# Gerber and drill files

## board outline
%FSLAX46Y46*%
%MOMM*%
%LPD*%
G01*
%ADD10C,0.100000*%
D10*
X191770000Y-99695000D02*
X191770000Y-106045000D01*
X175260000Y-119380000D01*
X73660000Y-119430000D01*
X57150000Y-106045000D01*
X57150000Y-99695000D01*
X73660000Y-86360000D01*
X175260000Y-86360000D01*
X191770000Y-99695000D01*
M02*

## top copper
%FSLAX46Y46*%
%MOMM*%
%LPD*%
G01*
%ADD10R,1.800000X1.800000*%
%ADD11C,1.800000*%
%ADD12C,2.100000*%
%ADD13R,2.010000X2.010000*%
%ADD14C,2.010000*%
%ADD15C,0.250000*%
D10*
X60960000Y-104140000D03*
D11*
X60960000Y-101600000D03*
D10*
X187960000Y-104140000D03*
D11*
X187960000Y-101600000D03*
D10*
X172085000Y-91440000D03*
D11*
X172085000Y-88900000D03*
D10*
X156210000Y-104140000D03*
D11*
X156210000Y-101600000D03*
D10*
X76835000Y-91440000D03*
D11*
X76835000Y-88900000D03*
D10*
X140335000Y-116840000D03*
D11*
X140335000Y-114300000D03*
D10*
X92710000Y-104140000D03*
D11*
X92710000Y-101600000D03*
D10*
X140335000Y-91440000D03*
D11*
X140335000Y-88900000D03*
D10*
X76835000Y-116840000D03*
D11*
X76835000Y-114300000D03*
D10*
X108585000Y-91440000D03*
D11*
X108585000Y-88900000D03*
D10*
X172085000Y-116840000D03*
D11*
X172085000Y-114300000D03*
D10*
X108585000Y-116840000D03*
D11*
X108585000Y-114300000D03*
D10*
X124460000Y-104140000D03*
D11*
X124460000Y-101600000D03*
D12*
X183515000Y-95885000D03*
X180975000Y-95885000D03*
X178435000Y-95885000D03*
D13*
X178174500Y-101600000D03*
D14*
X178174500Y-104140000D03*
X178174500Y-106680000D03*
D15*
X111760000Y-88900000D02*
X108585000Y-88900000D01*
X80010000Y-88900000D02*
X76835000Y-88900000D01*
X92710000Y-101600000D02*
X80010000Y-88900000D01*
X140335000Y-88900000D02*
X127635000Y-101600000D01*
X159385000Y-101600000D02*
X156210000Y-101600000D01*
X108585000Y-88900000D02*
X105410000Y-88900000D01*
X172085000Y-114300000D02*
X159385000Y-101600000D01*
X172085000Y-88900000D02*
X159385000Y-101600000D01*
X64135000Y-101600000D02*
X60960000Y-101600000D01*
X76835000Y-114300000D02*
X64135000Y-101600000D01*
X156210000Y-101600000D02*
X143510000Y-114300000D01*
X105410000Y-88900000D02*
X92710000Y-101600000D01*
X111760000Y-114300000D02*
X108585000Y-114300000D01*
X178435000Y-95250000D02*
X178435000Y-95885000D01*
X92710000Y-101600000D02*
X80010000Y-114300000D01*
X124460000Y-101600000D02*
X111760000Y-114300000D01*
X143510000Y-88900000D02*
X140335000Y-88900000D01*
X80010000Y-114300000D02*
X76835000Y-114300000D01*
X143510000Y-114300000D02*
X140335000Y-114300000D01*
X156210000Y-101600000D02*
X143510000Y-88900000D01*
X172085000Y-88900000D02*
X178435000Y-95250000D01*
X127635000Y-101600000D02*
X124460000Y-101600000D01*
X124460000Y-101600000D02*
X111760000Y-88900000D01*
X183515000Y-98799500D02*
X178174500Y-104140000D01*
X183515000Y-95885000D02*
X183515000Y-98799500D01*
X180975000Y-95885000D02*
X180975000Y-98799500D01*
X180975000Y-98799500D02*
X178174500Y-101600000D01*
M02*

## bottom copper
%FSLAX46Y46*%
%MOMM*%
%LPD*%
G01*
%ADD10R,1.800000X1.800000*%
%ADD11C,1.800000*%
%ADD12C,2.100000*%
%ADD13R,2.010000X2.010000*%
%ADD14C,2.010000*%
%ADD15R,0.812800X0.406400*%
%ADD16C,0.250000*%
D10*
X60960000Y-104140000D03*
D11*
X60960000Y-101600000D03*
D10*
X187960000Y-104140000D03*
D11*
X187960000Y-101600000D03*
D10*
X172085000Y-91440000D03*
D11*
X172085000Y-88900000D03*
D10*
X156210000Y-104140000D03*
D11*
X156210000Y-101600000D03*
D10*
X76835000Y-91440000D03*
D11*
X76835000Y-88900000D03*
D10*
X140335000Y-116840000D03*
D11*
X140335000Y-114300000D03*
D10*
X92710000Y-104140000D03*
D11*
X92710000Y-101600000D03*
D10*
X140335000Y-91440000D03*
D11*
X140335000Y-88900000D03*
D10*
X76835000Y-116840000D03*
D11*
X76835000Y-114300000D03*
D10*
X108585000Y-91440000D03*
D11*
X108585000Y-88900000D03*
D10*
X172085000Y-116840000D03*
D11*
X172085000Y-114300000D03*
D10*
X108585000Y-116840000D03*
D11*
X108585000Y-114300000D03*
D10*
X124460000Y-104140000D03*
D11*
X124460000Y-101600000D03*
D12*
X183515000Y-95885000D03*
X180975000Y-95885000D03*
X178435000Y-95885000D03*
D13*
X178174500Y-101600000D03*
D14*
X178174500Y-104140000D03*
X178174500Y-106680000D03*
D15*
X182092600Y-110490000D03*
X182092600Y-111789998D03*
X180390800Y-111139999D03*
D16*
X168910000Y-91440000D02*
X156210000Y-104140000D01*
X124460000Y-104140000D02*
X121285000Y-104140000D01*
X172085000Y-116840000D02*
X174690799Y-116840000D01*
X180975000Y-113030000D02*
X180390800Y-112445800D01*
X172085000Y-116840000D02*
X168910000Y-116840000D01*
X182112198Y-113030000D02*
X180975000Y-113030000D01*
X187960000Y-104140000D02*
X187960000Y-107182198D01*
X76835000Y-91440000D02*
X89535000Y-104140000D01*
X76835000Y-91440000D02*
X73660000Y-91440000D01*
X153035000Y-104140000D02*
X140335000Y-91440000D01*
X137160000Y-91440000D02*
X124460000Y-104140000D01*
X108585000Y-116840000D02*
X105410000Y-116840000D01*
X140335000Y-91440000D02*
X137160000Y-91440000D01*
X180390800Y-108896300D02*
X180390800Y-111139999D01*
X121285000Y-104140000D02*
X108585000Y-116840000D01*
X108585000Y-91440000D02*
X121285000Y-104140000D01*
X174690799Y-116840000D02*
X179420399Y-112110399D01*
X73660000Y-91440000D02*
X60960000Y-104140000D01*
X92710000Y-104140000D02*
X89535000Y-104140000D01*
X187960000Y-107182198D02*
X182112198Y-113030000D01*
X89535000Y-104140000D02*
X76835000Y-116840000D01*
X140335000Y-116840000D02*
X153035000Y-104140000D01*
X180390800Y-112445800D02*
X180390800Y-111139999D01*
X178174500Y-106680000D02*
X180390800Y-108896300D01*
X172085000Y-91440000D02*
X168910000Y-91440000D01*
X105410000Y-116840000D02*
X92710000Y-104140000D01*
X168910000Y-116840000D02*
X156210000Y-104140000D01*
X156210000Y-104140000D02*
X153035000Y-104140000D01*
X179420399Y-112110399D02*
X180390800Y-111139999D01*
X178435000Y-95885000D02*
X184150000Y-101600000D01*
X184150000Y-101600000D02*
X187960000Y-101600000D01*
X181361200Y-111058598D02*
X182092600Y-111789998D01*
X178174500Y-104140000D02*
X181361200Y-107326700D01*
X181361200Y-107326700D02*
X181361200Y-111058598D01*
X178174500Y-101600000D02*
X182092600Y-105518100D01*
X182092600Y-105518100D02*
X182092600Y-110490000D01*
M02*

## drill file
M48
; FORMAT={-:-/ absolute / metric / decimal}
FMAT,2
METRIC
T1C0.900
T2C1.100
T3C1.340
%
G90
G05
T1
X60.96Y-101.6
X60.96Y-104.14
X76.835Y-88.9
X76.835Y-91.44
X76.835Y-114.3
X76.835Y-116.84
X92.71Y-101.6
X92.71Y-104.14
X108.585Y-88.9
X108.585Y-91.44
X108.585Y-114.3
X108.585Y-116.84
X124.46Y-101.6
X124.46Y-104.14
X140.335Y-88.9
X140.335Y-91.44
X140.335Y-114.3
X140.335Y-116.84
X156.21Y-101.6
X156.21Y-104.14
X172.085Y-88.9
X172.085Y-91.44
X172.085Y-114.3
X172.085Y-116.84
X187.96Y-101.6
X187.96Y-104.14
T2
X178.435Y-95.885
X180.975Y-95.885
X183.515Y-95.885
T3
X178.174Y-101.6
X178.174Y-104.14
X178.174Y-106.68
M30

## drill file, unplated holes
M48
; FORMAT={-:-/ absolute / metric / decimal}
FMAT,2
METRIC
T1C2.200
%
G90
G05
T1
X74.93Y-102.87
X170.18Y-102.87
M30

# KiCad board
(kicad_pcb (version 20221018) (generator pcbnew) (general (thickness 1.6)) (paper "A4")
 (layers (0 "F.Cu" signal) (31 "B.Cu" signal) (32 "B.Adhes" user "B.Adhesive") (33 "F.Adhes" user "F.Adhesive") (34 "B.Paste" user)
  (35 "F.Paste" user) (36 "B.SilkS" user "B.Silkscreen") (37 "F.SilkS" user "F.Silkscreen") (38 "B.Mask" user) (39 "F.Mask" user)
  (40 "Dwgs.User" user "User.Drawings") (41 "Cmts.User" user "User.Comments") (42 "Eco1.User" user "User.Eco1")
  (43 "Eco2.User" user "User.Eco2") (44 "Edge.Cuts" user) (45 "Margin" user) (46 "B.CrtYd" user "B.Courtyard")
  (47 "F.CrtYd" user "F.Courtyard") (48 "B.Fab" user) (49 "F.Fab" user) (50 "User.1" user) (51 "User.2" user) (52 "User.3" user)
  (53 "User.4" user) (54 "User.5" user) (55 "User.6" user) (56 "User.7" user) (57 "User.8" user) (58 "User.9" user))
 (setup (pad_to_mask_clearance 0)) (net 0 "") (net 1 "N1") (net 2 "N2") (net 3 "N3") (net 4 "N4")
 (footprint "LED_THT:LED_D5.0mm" (layer "F.Cu") (at 60.96 104.14 90)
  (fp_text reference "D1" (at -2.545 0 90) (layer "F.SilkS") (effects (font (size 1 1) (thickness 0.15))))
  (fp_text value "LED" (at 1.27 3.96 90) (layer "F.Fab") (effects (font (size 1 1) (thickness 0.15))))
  (pad "1" thru_hole rect (at 0 0 90) (size 1.8 1.8) (drill 0.9) (layers "*.Cu" "*.Mask") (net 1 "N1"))
  (pad "2" thru_hole circle (at 2.54 0 90) (size 1.8 1.8) (drill 0.9) (layers "*.Cu" "*.Mask") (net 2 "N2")))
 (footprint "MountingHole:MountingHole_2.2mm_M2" (layer "F.Cu") (at 170.18 102.87 90)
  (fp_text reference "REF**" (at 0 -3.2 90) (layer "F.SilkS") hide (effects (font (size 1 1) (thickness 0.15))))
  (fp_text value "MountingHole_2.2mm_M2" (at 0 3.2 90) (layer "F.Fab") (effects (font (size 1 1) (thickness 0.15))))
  (pad "" np_thru_hole circle (at 0 0 90) (size 2.2 2.2) (drill 2.2) (layers "F&B.Cu" "*.Mask")))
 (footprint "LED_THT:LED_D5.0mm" (layer "F.Cu") (at 187.96 104.14 90)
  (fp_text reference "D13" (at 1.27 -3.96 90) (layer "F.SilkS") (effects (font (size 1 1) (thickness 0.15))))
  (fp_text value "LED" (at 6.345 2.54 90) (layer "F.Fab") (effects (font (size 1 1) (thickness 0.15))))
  (pad "1" thru_hole rect (at 0 0 90) (size 1.8 1.8) (drill 0.9) (layers "*.Cu" "*.Mask") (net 1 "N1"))
  (pad "2" thru_hole circle (at 2.54 0 90) (size 1.8 1.8) (drill 0.9) (layers "*.Cu" "*.Mask") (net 2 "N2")))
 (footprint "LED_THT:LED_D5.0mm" (layer "F.Cu") (at 172.085 91.44 90)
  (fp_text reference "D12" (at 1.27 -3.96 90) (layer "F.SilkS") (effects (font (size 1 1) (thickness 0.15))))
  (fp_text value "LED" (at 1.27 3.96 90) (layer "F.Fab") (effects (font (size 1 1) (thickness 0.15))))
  (pad "1" thru_hole rect (at 0 0 90) (size 1.8 1.8) (drill 0.9) (layers "*.Cu" "*.Mask") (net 1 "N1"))
  (pad "2" thru_hole circle (at 2.54 0 90) (size 1.8 1.8) (drill 0.9) (layers "*.Cu" "*.Mask") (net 2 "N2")))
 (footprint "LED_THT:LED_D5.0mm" (layer "F.Cu") (at 156.21 104.14 90)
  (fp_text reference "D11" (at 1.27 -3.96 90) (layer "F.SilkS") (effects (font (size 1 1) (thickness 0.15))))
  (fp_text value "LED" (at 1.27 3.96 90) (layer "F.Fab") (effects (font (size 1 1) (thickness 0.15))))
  (pad "1" thru_hole rect (at 0 0 90) (size 1.8 1.8) (drill 0.9) (layers "*.Cu" "*.Mask") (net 1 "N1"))
  (pad "2" thru_hole circle (at 2.54 0 90) (size 1.8 1.8) (drill 0.9) (layers "*.Cu" "*.Mask") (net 2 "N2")))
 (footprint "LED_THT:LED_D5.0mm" (layer "F.Cu") (at 76.835 91.44 90)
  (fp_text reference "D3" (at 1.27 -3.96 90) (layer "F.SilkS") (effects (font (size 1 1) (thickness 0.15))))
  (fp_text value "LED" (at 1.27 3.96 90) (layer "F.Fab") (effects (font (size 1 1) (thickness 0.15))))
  (pad "1" thru_hole rect (at 0 0 90) (size 1.8 1.8) (drill 0.9) (layers "*.Cu" "*.Mask") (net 1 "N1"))
  (pad "2" thru_hole circle (at 2.54 0 90) (size 1.8 1.8) (drill 0.9) (layers "*.Cu" "*.Mask") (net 2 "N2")))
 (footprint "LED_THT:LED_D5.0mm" (layer "F.Cu") (at 140.335 116.84 90)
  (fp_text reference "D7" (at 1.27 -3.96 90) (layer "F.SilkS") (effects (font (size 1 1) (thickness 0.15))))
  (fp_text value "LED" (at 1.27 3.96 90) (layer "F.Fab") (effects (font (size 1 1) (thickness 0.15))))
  (pad "1" thru_hole rect (at 0 0 90) (size 1.8 1.8) (drill 0.9) (layers "*.Cu" "*.Mask") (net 1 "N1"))
  (pad "2" thru_hole circle (at 2.54 0 90) (size 1.8 1.8) (drill 0.9) (layers "*.Cu" "*.Mask") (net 2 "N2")))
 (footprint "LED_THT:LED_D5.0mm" (layer "F.Cu") (at 92.71 104.14 90)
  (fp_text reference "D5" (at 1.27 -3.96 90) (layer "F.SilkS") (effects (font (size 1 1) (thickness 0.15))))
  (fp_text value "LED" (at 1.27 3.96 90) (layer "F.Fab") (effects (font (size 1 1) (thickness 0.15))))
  (pad "1" thru_hole rect (at 0 0 90) (size 1.8 1.8) (drill 0.9) (layers "*.Cu" "*.Mask") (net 1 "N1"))
  (pad "2" thru_hole circle (at 2.54 0 90) (size 1.8 1.8) (drill 0.9) (layers "*.Cu" "*.Mask") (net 2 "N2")))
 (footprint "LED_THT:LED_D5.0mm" (layer "F.Cu") (at 140.335 91.44 90)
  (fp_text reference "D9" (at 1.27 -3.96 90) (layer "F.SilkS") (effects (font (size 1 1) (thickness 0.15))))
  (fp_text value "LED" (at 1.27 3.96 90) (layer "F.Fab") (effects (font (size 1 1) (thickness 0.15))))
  (pad "1" thru_hole rect (at 0 0 90) (size 1.8 1.8) (drill 0.9) (layers "*.Cu" "*.Mask") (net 1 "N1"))
  (pad "2" thru_hole circle (at 2.54 0 90) (size 1.8 1.8) (drill 0.9) (layers "*.Cu" "*.Mask") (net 2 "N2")))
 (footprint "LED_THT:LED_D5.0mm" (layer "F.Cu") (at 76.835 116.84 90)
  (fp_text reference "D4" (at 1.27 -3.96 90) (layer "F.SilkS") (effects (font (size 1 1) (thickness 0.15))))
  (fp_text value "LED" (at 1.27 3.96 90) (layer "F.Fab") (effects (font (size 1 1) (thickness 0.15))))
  (pad "1" thru_hole rect (at 0 0 90) (size 1.8 1.8) (drill 0.9) (layers "*.Cu" "*.Mask") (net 1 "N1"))
  (pad "2" thru_hole circle (at 2.54 0 90) (size 1.8 1.8) (drill 0.9) (layers "*.Cu" "*.Mask") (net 2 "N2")))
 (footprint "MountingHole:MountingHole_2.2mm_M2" (layer "F.Cu") (at 74.93 102.87 90)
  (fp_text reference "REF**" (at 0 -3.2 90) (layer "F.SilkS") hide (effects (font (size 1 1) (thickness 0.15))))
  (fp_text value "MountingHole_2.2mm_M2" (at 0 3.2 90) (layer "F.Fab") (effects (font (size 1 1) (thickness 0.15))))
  (pad "" np_thru_hole circle (at 0 0 90) (size 2.2 2.2) (drill 2.2) (layers "*.Cu" "*.Mask")))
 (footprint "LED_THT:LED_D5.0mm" (layer "F.Cu") (at 108.585 91.44 90)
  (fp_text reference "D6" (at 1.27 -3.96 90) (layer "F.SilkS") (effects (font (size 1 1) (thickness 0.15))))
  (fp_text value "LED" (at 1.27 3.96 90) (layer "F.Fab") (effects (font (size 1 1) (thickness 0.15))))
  (pad "1" thru_hole rect (at 0 0 90) (size 1.8 1.8) (drill 0.9) (layers "*.Cu" "*.Mask") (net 1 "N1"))
  (pad "2" thru_hole circle (at 2.54 0 90) (size 1.8 1.8) (drill 0.9) (layers "*.Cu" "*.Mask") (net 2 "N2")))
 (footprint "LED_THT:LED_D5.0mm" (layer "F.Cu") (at 172.085 116.84 90)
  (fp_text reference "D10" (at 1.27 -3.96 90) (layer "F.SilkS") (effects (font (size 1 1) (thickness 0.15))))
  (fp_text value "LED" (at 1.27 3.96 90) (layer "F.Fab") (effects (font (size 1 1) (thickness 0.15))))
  (pad "1" thru_hole rect (at 0 0 90) (size 1.8 1.8) (drill 0.9) (layers "*.Cu" "*.Mask") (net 1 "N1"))
  (pad "2" thru_hole circle (at 2.54 0 90) (size 1.8 1.8) (drill 0.9) (layers "*.Cu" "*.Mask") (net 2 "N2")))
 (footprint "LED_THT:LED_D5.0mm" (layer "F.Cu") (at 108.585 116.84 90)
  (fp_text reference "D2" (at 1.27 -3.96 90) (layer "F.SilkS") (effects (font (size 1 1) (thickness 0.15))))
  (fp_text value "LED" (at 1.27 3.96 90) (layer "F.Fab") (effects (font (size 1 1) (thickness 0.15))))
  (pad "1" thru_hole rect (at 0 0 90) (size 1.8 1.8) (drill 0.9) (layers "*.Cu" "*.Mask") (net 1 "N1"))
  (pad "2" thru_hole circle (at 2.54 0 90) (size 1.8 1.8) (drill 0.9) (layers "*.Cu" "*.Mask") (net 2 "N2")))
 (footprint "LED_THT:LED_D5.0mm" (layer "F.Cu") (at 124.46 104.14 90)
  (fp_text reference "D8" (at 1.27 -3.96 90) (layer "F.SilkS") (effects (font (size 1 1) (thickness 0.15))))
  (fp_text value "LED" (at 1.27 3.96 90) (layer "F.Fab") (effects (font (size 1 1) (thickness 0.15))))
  (pad "1" thru_hole rect (at 0 0 90) (size 1.8 1.8) (drill 0.9) (layers "*.Cu" "*.Mask") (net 1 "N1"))
  (pad "2" thru_hole circle (at 2.54 0 90) (size 1.8 1.8) (drill 0.9) (layers "*.Cu" "*.Mask") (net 2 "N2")))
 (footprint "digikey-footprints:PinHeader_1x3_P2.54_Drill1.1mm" (layer "B.Cu") (at 183.515 95.885 180)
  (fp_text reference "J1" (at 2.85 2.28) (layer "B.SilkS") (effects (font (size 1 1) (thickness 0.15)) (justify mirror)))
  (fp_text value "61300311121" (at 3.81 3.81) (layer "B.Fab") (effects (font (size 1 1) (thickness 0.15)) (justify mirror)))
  (pad "1" thru_hole circle (at 0 0 180) (size 2.1 2.1) (drill 1.1) (layers "*.Cu" "*.Mask") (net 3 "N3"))
  (pad "2" thru_hole circle (at 2.54 0 180) (size 2.1 2.1) (drill 1.1) (layers "*.Cu" "*.Mask") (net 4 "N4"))
  (pad "3" thru_hole circle (at 5.08 0 180) (size 2.1 2.1) (drill 1.1) (layers "*.Cu" "*.Mask") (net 2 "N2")))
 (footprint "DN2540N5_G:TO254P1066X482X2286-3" (layer "B.Cu") (at 178.1745 101.6 -90)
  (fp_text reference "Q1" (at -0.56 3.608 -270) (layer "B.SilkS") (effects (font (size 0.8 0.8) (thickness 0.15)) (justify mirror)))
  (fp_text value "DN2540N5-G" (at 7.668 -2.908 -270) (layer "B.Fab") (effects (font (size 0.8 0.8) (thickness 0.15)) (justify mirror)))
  (pad "1" thru_hole rect (at 0 0 270) (size 2.01 2.01) (drill 1.34) (layers "*.Cu" "*.Mask") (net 4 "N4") (solder_mask_margin 0.102))
  (pad "2" thru_hole circle (at 2.54 0 270) (size 2.01 2.01) (drill 1.34) (layers "*.Cu" "*.Mask") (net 3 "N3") (solder_mask_margin 0.102))
  (pad "3" thru_hole circle (at 5.08 0 270) (size 2.01 2.01) (drill 1.34) (layers "*.Cu" "*.Mask") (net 1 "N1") (solder_mask_margin 0.102)))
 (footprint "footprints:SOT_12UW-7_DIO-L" (layer "B.Cu") (at 181.2417 111.139999 -90)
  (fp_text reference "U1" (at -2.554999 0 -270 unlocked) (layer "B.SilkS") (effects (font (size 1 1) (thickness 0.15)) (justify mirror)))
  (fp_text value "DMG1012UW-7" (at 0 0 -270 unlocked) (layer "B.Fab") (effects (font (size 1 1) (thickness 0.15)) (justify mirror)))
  (pad "1" smd rect (at -0.649999 -0.8509 270) (size 0.4064 0.8128) (layers "B.Cu" "B.Paste" "B.Mask") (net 4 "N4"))
  (pad "2" smd rect (at 0.649999 -0.8509 270) (size 0.4064 0.8128) (layers "B.Cu" "B.Paste" "B.Mask") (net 3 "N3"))
  (pad "3" smd rect (at 0 0.8509 270) (size 0.4064 0.8128) (layers "B.Cu" "B.Paste" "B.Mask") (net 1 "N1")))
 (gr_poly
  (pts (xy 57.15 99.695) (xy 73.66 86.36) (xy 175.26 86.36) (xy 191.77 99.695) (xy 191.77 106.045) (xy 175.26 119.38) (xy 73.66 119.43)
   (xy 57.15 106.045))
  (stroke (width 0.1) (type solid)) (fill none) (layer "Edge.Cuts"))
 (segment (start 168.91 91.44) (end 156.21 104.14) (width 0.25) (layer "B.Cu") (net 1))
 (segment (start 124.46 104.14) (end 121.285 104.14) (width 0.25) (layer "B.Cu") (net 1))
 (segment (start 172.085 116.84) (end 174.690799 116.84) (width 0.25) (layer "B.Cu") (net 1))
 (segment (start 180.975 113.03) (end 180.3908 112.4458) (width 0.25) (layer "B.Cu") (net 1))
 (segment (start 172.085 116.84) (end 168.91 116.84) (width 0.25) (layer "B.Cu") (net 1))
 (segment (start 182.112198 113.03) (end 180.975 113.03) (width 0.25) (layer "B.Cu") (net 1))
 (segment (start 187.96 104.14) (end 187.96 107.182198) (width 0.25) (layer "B.Cu") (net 1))
 (segment (start 76.835 91.44) (end 89.535 104.14) (width 0.25) (layer "B.Cu") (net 1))
 (segment (start 76.835 91.44) (end 73.66 91.44) (width 0.25) (layer "B.Cu") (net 1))
 (segment (start 153.035 104.14) (end 140.335 91.44) (width 0.25) (layer "B.Cu") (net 1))
 (segment (start 137.16 91.44) (end 124.46 104.14) (width 0.25) (layer "B.Cu") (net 1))
 (segment (start 108.585 116.84) (end 105.41 116.84) (width 0.25) (layer "B.Cu") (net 1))
 (segment (start 140.335 91.44) (end 137.16 91.44) (width 0.25) (layer "B.Cu") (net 1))
 (segment (start 180.3908 108.8963) (end 180.3908 111.139999) (width 0.25) (layer "B.Cu") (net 1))
 (segment (start 121.285 104.14) (end 108.585 116.84) (width 0.25) (layer "B.Cu") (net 1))
 (segment (start 108.585 91.44) (end 121.285 104.14) (width 0.25) (layer "B.Cu") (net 1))
 (segment (start 174.690799 116.84) (end 179.420399 112.110399) (width 0.25) (layer "B.Cu") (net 1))
 (segment (start 73.66 91.44) (end 60.96 104.14) (width 0.25) (layer "B.Cu") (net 1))
 (segment (start 92.71 104.14) (end 89.535 104.14) (width 0.25) (layer "B.Cu") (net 1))
 (segment (start 187.96 107.182198) (end 182.112198 113.03) (width 0.25) (layer "B.Cu") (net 1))
 (segment (start 89.535 104.14) (end 76.835 116.84) (width 0.25) (layer "B.Cu") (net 1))
 (segment (start 140.335 116.84) (end 153.035 104.14) (width 0.25) (layer "B.Cu") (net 1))
 (segment (start 180.3908 112.4458) (end 180.3908 111.139999) (width 0.25) (layer "B.Cu") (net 1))
 (segment (start 178.1745 106.68) (end 180.3908 108.8963) (width 0.25) (layer "B.Cu") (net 1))
 (segment (start 172.085 91.44) (end 168.91 91.44) (width 0.25) (layer "B.Cu") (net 1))
 (segment (start 105.41 116.84) (end 92.71 104.14) (width 0.25) (layer "B.Cu") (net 1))
 (segment (start 168.91 116.84) (end 156.21 104.14) (width 0.25) (layer "B.Cu") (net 1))
 (segment (start 156.21 104.14) (end 153.035 104.14) (width 0.25) (layer "B.Cu") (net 1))
 (segment (start 179.420399 112.110399) (end 180.3908 111.139999) (width 0.25) (layer "B.Cu") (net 1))
 (segment (start 111.76 88.9) (end 108.585 88.9) (width 0.25) (layer "F.Cu") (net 2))
 (segment (start 80.01 88.9) (end 76.835 88.9) (width 0.25) (layer "F.Cu") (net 2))
 (segment (start 92.71 101.6) (end 80.01 88.9) (width 0.25) (layer "F.Cu") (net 2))
 (segment (start 140.335 88.9) (end 127.635 101.6) (width 0.25) (layer "F.Cu") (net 2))
 (segment (start 159.385 101.6) (end 156.21 101.6) (width 0.25) (layer "F.Cu") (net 2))
 (segment (start 108.585 88.9) (end 105.41 88.9) (width 0.25) (layer "F.Cu") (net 2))
 (segment (start 172.085 114.3) (end 159.385 101.6) (width 0.25) (layer "F.Cu") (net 2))
 (segment (start 172.085 88.9) (end 159.385 101.6) (width 0.25) (layer "F.Cu") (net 2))
 (segment (start 64.135 101.6) (end 60.96 101.6) (width 0.25) (layer "F.Cu") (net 2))
 (segment (start 76.835 114.3) (end 64.135 101.6) (width 0.25) (layer "F.Cu") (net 2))
 (segment (start 156.21 101.6) (end 143.51 114.3) (width 0.25) (layer "F.Cu") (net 2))
 (segment (start 105.41 88.9) (end 92.71 101.6) (width 0.25) (layer "F.Cu") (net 2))
 (segment (start 111.76 114.3) (end 108.585 114.3) (width 0.25) (layer "F.Cu") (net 2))
 (segment (start 178.435 95.25) (end 178.435 95.885) (width 0.25) (layer "F.Cu") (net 2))
 (segment (start 92.71 101.6) (end 80.01 114.3) (width 0.25) (layer "F.Cu") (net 2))
 (segment (start 124.46 101.6) (end 111.76 114.3) (width 0.25) (layer "F.Cu") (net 2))
 (segment (start 143.51 88.9) (end 140.335 88.9) (width 0.25) (layer "F.Cu") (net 2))
 (segment (start 80.01 114.3) (end 76.835 114.3) (width 0.25) (layer "F.Cu") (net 2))
 (segment (start 143.51 114.3) (end 140.335 114.3) (width 0.25) (layer "F.Cu") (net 2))
 (segment (start 156.21 101.6) (end 143.51 88.9) (width 0.25) (layer "F.Cu") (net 2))
 (segment (start 172.085 88.9) (end 178.435 95.25) (width 0.25) (layer "F.Cu") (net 2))
 (segment (start 127.635 101.6) (end 124.46 101.6) (width 0.25) (layer "F.Cu") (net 2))
 (segment (start 124.46 101.6) (end 111.76 88.9) (width 0.25) (layer "F.Cu") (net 2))
 (segment (start 178.435 95.885) (end 184.15 101.6) (width 0.25) (layer "B.Cu") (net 2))
 (segment (start 184.15 101.6) (end 187.96 101.6) (width 0.25) (layer "B.Cu") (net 2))
 (segment (start 183.515 98.7995) (end 178.1745 104.14) (width 0.25) (layer "F.Cu") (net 3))
 (segment (start 183.515 95.885) (end 183.515 98.7995) (width 0.25) (layer "F.Cu") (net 3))
 (segment (start 181.3612 111.058598) (end 182.0926 111.789998) (width 0.25) (layer "B.Cu") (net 3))
 (segment (start 178.1745 104.14) (end 181.3612 107.3267) (width 0.25) (layer "B.Cu") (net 3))
 (segment (start 181.3612 107.3267) (end 181.3612 111.058598) (width 0.25) (layer "B.Cu") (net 3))
 (segment (start 180.975 95.885) (end 180.975 98.7995) (width 0.25) (layer "F.Cu") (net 4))
 (segment (start 180.975 98.7995) (end 178.1745 101.6) (width 0.25) (layer "F.Cu") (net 4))
 (segment (start 178.1745 101.6) (end 182.0926 105.5181) (width 0.25) (layer "B.Cu") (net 4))
 (segment (start 182.0926 105.5181) (end 182.0926 110.49) (width 0.25) (layer "B.Cu") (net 4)))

